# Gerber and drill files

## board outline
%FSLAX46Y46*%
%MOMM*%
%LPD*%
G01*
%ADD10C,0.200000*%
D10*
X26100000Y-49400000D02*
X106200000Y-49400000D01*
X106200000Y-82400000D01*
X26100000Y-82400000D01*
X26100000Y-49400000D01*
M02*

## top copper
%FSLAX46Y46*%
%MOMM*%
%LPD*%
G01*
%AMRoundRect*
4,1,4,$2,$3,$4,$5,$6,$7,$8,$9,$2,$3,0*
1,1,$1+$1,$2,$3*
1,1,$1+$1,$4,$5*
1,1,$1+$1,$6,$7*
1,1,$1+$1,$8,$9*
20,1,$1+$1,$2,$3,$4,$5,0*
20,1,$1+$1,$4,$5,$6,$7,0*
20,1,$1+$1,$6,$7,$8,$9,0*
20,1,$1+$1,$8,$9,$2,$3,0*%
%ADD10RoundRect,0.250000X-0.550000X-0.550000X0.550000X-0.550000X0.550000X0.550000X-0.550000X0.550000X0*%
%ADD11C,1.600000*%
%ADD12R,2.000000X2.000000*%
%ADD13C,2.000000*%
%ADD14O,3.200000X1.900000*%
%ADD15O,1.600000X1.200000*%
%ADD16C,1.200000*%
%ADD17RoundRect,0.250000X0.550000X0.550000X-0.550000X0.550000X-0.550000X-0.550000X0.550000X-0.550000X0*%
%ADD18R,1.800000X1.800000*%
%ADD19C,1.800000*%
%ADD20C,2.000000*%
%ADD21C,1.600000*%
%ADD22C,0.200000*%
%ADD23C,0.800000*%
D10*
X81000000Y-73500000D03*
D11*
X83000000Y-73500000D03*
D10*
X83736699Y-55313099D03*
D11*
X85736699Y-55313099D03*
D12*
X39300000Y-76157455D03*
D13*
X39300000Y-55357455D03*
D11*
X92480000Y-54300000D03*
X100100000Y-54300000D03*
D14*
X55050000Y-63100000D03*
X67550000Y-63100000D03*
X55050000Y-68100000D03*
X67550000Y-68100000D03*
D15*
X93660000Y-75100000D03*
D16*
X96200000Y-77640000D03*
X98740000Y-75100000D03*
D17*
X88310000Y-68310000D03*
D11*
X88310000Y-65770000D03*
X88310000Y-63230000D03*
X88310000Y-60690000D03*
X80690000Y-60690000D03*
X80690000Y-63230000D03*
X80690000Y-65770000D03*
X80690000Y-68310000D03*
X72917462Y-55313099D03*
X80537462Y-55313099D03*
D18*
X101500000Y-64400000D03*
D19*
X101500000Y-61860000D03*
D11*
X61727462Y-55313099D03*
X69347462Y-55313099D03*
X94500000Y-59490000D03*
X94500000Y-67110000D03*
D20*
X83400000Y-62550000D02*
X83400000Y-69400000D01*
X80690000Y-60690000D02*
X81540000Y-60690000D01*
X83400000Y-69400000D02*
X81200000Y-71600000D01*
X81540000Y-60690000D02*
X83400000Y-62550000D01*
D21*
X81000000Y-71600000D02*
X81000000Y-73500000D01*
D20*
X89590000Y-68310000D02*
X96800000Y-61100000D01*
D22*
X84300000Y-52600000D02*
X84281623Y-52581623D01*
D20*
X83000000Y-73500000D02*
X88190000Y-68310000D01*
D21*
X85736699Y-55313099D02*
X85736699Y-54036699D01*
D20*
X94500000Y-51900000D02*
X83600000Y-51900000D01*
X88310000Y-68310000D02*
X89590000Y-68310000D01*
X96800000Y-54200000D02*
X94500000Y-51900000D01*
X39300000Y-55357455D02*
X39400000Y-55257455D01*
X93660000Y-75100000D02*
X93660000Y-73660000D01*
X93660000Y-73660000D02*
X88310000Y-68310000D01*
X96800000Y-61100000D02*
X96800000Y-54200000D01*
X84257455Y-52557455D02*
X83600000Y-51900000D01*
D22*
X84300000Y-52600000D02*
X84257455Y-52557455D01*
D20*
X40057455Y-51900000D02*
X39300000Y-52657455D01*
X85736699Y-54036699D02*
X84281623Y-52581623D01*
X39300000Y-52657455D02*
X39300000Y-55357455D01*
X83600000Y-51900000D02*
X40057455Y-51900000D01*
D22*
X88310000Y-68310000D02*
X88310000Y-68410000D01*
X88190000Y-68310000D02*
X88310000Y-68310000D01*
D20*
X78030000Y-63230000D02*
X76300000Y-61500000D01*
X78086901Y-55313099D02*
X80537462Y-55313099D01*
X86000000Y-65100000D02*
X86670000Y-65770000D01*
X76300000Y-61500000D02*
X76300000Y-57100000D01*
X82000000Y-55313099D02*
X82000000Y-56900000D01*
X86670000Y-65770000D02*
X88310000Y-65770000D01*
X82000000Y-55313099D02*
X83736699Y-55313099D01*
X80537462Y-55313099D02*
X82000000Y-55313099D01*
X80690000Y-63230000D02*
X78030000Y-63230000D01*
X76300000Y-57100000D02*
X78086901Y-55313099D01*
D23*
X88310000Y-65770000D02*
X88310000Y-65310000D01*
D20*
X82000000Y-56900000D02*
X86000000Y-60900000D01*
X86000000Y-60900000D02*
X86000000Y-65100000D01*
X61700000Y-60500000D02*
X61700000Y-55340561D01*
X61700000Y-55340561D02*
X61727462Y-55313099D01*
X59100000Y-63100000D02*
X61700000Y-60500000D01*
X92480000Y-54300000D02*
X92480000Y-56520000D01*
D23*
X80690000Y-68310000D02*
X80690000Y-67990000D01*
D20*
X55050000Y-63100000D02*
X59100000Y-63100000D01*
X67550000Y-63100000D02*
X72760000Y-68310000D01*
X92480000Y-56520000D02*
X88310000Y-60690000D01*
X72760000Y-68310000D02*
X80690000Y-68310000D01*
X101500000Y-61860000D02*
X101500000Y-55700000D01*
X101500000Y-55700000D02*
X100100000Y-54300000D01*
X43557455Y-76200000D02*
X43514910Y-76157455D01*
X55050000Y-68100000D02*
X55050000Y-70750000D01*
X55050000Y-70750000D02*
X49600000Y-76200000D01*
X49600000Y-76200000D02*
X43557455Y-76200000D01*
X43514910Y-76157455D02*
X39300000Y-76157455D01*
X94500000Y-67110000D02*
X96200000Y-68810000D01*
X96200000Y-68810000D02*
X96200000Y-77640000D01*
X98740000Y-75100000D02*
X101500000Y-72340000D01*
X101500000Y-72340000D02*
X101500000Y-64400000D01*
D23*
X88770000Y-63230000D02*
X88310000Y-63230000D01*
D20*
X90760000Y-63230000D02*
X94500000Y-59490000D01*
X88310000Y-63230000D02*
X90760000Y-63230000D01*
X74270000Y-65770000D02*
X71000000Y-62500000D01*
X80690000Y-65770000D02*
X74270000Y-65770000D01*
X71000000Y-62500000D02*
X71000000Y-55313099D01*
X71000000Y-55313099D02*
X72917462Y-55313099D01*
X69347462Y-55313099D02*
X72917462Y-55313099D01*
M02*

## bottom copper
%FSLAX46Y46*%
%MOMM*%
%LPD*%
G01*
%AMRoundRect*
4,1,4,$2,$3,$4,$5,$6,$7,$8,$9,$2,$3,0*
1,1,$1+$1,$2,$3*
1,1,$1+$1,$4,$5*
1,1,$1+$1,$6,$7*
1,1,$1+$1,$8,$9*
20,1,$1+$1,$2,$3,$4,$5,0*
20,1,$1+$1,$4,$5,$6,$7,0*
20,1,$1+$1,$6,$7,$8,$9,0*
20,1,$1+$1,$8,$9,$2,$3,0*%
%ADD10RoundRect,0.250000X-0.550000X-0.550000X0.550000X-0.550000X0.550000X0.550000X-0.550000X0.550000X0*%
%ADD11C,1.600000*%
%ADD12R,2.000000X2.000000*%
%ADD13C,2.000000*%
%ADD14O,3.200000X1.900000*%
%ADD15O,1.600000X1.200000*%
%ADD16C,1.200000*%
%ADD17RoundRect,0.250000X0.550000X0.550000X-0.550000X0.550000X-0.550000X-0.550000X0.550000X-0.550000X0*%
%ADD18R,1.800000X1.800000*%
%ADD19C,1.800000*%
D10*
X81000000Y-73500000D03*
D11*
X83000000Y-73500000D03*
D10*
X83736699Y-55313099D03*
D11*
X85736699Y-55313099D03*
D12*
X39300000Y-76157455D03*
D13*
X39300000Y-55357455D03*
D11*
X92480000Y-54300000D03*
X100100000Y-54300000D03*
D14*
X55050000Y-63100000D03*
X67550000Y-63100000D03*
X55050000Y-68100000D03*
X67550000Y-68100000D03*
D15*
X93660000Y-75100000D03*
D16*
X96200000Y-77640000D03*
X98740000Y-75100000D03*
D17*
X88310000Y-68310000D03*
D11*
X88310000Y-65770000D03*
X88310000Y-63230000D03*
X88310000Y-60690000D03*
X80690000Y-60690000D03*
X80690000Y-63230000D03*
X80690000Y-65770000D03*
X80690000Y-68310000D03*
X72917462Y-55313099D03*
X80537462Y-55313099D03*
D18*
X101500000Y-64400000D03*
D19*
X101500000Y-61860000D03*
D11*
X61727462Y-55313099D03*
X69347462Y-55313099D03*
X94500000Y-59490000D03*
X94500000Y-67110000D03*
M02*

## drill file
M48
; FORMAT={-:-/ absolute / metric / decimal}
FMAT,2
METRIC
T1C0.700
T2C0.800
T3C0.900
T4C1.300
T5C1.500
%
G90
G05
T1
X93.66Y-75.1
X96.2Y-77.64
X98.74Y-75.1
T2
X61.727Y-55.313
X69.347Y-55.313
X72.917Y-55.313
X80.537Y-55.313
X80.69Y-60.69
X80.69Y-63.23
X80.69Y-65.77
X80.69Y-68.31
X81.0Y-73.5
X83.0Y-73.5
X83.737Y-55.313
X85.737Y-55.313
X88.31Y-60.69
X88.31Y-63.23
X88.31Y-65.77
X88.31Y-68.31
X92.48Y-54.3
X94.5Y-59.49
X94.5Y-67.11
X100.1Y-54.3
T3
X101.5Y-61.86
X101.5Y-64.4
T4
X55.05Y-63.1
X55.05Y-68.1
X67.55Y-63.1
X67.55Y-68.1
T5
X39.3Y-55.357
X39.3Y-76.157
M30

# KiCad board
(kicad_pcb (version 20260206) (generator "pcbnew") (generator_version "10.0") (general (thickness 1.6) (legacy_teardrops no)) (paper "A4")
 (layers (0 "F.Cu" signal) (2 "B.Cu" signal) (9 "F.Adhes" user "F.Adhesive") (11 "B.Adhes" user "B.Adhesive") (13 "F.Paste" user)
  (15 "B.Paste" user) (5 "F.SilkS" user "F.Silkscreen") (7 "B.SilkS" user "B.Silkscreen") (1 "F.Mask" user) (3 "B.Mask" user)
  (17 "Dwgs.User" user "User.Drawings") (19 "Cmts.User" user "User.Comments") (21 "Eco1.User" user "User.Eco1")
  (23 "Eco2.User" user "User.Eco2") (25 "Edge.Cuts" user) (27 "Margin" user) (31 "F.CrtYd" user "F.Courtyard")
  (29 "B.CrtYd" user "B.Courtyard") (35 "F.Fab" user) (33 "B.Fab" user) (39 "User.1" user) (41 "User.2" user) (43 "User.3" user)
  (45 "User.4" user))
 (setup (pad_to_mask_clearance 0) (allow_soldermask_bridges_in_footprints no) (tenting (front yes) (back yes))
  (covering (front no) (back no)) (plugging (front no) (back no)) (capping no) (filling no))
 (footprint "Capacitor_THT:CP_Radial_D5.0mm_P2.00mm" (layer "F.Cu") (at 81 73.5)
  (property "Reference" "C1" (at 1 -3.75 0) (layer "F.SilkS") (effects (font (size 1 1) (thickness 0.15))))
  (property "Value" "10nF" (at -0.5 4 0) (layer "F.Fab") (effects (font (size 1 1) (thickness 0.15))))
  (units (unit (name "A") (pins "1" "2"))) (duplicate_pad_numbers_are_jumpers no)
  (pad "1" thru_hole roundrect (at 0 0) (size 1.6 1.6) (drill 0.8) (layers "*.Cu" "*.Mask") (remove_unused_layers no)
   (roundrect_rratio 0.15625) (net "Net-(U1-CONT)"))
  (pad "2" thru_hole circle (at 2 0) (size 1.6 1.6) (drill 0.8) (layers "*.Cu" "*.Mask") (remove_unused_layers no) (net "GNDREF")))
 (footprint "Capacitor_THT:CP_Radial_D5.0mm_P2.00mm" (layer "F.Cu") (at 83.736699 55.313099)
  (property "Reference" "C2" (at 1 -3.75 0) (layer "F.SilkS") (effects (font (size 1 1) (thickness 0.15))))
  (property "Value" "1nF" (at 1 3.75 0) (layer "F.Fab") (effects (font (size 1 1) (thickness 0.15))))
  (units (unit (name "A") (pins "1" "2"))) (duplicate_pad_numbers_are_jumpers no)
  (pad "1" thru_hole roundrect (at 0 0) (size 1.6 1.6) (drill 0.8) (layers "*.Cu" "*.Mask") (remove_unused_layers no)
   (roundrect_rratio 0.15625) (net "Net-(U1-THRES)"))
  (pad "2" thru_hole circle (at 2 0) (size 1.6 1.6) (drill 0.8) (layers "*.Cu" "*.Mask") (remove_unused_layers no) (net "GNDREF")))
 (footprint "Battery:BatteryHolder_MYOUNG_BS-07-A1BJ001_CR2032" (layer "F.Cu") (at 39.3 76.157455 90)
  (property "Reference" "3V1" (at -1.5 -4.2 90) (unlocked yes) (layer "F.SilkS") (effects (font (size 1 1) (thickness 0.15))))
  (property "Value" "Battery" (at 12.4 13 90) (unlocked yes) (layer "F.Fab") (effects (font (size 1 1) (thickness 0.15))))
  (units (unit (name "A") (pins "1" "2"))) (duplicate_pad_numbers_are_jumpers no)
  (pad "1" thru_hole rect (at 0 0 270) (size 2 2) (drill 1.5) (layers "*.Cu" "*.Mask") (remove_unused_layers no) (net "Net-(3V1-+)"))
  (pad "2" thru_hole circle (at 20.8 0 270) (size 2 2) (drill 1.5) (layers "*.Cu" "*.Mask") (remove_unused_layers no) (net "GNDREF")))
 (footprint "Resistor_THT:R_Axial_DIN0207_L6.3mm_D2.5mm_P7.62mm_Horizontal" (layer "F.Cu") (at 92.48 54.3)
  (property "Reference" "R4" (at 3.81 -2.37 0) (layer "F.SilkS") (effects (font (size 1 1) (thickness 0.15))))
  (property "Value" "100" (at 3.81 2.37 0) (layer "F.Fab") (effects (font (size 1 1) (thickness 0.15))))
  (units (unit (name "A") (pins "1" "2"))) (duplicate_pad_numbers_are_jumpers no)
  (pad "1" thru_hole circle (at 0 0) (size 1.6 1.6) (drill 0.8) (layers "*.Cu" "*.Mask") (remove_unused_layers no) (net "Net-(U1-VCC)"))
  (pad "2" thru_hole circle (at 7.62 0) (size 1.6 1.6) (drill 0.8) (layers "*.Cu" "*.Mask") (remove_unused_layers no) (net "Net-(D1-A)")))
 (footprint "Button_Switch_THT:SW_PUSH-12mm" (layer "F.Cu") (at 55.05 63.1)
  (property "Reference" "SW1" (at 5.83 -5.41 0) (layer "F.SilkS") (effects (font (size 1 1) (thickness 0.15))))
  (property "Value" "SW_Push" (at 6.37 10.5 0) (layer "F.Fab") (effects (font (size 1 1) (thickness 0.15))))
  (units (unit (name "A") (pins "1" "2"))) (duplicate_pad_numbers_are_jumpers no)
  (pad "1" thru_hole oval (at 0 0) (size 3.2 1.9) (drill 1.3) (layers "*.Cu" "*.Mask") (remove_unused_layers no) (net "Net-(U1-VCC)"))
  (pad "1" thru_hole oval (at 12.5 0) (size 3.2 1.9) (drill 1.3) (layers "*.Cu" "*.Mask") (remove_unused_layers no) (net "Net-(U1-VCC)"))
  (pad "2" thru_hole oval (at 0 5) (size 3.2 1.9) (drill 1.3) (layers "*.Cu" "*.Mask") (remove_unused_layers no) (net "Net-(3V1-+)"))
  (pad "2" thru_hole oval (at 12.5 5) (size 3.2 1.9) (drill 1.3) (layers "*.Cu" "*.Mask") (remove_unused_layers no) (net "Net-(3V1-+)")))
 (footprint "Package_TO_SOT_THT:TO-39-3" (layer "F.Cu") (at 93.66 75.1)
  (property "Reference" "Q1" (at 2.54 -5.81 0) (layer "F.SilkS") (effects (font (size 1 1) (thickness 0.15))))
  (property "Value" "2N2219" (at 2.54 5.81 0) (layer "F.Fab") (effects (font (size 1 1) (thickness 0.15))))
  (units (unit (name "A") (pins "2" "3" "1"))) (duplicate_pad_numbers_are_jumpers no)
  (pad "1" thru_hole oval (at 0 0) (size 1.6 1.2) (drill 0.7) (layers "*.Cu" "*.Mask") (remove_unused_layers no) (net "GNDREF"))
  (pad "2" thru_hole circle (at 2.54 2.54) (size 1.2 1.2) (drill 0.7) (layers "*.Cu" "*.Mask") (remove_unused_layers no) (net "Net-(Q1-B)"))
  (pad "3" thru_hole circle (at 5.08 0) (size 1.2 1.2) (drill 0.7) (layers "*.Cu" "*.Mask") (remove_unused_layers no) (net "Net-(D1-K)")))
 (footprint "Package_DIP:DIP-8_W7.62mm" (layer "F.Cu") (at 88.31 68.31 180)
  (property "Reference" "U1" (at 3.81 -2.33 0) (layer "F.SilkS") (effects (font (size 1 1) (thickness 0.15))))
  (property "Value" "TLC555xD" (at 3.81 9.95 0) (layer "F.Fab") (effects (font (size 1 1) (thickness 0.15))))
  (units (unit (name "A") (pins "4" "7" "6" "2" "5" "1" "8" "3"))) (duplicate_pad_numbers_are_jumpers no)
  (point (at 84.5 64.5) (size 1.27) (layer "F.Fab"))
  (pad "1" thru_hole roundrect (at 0 0 180) (size 1.6 1.6) (drill 0.8) (layers "*.Cu" "*.Mask") (remove_unused_layers no)
   (roundrect_rratio 0.15625) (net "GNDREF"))
  (pad "2" thru_hole circle (at 0 2.54 180) (size 1.6 1.6) (drill 0.8) (layers "*.Cu" "*.Mask") (remove_unused_layers no)
   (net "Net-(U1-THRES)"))
  (pad "3" thru_hole circle (at 0 5.08 180) (size 1.6 1.6) (drill 0.8) (layers "*.Cu" "*.Mask") (remove_unused_layers no)
   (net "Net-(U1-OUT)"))
  (pad "4" thru_hole circle (at 0 7.62 180) (size 1.6 1.6) (drill 0.8) (layers "*.Cu" "*.Mask") (remove_unused_layers no)
   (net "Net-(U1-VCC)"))
  (pad "5" thru_hole circle (at 7.62 7.62 180) (size 1.6 1.6) (drill 0.8) (layers "*.Cu" "*.Mask") (remove_unused_layers no)
   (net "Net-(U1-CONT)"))
  (pad "6" thru_hole circle (at 7.62 5.08 180) (size 1.6 1.6) (drill 0.8) (layers "*.Cu" "*.Mask") (remove_unused_layers no)
   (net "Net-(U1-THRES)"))
  (pad "7" thru_hole circle (at 7.62 2.54 180) (size 1.6 1.6) (drill 0.8) (layers "*.Cu" "*.Mask") (remove_unused_layers no)
   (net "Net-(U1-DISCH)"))
  (pad "8" thru_hole circle (at 7.62 0 180) (size 1.6 1.6) (drill 0.8) (layers "*.Cu" "*.Mask") (remove_unused_layers no)
   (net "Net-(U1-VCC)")))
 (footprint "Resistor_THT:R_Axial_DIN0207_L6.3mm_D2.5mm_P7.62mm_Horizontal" (layer "F.Cu") (at 72.917462 55.313099)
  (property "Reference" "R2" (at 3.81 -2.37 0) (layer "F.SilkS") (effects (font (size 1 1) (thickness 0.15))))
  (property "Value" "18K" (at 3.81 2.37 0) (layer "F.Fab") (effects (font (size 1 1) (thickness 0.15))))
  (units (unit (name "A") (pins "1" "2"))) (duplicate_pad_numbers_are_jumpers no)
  (pad "1" thru_hole circle (at 0 0) (size 1.6 1.6) (drill 0.8) (layers "*.Cu" "*.Mask") (remove_unused_layers no) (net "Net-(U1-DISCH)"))
  (pad "2" thru_hole circle (at 7.62 0) (size 1.6 1.6) (drill 0.8) (layers "*.Cu" "*.Mask") (remove_unused_layers no) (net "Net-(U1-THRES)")))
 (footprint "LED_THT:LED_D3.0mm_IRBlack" (layer "F.Cu") (at 101.5 64.4 90)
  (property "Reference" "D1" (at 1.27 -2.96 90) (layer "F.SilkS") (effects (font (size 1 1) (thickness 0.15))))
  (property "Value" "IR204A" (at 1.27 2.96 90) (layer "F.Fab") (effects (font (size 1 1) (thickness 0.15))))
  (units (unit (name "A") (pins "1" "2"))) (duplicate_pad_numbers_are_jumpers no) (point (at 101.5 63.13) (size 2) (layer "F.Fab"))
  (pad "1" thru_hole rect (at 0 0 90) (size 1.8 1.8) (drill 0.9) (layers "*.Cu" "*.Mask") (remove_unused_layers no) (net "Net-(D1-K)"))
  (pad "2" thru_hole circle (at 2.54 0 90) (size 1.8 1.8) (drill 0.9) (layers "*.Cu" "*.Mask") (remove_unused_layers no) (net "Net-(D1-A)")))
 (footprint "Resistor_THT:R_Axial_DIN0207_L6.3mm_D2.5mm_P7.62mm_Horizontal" (layer "F.Cu") (at 61.727462 55.313099)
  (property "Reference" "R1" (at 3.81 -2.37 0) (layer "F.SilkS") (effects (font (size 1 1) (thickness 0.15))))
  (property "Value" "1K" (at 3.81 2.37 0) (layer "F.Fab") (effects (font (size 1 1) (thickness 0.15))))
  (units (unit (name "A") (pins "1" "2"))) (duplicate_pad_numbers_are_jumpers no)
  (pad "1" thru_hole circle (at 0 0) (size 1.6 1.6) (drill 0.8) (layers "*.Cu" "*.Mask") (remove_unused_layers no) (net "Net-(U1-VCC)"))
  (pad "2" thru_hole circle (at 7.62 0) (size 1.6 1.6) (drill 0.8) (layers "*.Cu" "*.Mask") (remove_unused_layers no) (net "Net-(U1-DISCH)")))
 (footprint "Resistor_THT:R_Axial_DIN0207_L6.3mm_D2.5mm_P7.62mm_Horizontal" (layer "F.Cu") (at 94.5 59.49 -90)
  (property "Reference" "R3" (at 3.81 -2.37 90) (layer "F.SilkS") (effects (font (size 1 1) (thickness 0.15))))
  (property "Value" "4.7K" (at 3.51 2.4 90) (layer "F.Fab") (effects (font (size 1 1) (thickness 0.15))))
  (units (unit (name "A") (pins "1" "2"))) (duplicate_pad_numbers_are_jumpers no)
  (pad "1" thru_hole circle (at 0 0 270) (size 1.6 1.6) (drill 0.8) (layers "*.Cu" "*.Mask") (remove_unused_layers no) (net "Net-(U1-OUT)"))
  (pad "2" thru_hole circle (at 7.62 0 270) (size 1.6 1.6) (drill 0.8) (layers "*.Cu" "*.Mask") (remove_unused_layers no) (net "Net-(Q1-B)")))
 (gr_rect (start 26.1 49.4) (end 106.2 82.4) (stroke (width 0.2) (type default)) (fill no) (layer "Edge.Cuts"))
 (segment (start 83.4 62.55) (end 83.4 69.4) (width 2) (layer "F.Cu") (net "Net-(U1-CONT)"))
 (segment (start 80.69 60.69) (end 81.54 60.69) (width 2) (layer "F.Cu") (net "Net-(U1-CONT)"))
 (segment (start 83.4 69.4) (end 81.2 71.6) (width 2) (layer "F.Cu") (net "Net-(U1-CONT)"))
 (segment (start 81.54 60.69) (end 83.4 62.55) (width 2) (layer "F.Cu") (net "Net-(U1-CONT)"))
 (segment (start 81 71.6) (end 81 73.5) (width 1.6) (layer "F.Cu") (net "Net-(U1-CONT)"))
 (segment (start 89.59 68.31) (end 96.8 61.1) (width 2) (layer "F.Cu") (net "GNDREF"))
 (segment (start 84.3 52.6) (end 84.281623 52.581623) (width 0.2) (layer "F.Cu") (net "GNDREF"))
 (segment (start 83 73.5) (end 88.19 68.31) (width 2) (layer "F.Cu") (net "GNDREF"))
 (segment (start 85.736699 55.313099) (end 85.736699 54.036699) (width 1.6) (layer "F.Cu") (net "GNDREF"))
 (segment (start 94.5 51.9) (end 83.6 51.9) (width 2) (layer "F.Cu") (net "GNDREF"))
 (segment (start 88.31 68.31) (end 89.59 68.31) (width 2) (layer "F.Cu") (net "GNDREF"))
 (segment (start 96.8 54.2) (end 94.5 51.9) (width 2) (layer "F.Cu") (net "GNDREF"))
 (segment (start 39.3 55.357455) (end 39.4 55.257455) (width 2) (layer "F.Cu") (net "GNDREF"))
 (segment (start 93.66 75.1) (end 93.66 73.66) (width 2) (layer "F.Cu") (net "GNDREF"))
 (segment (start 93.66 73.66) (end 88.31 68.31) (width 2) (layer "F.Cu") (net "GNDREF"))
 (segment (start 96.8 61.1) (end 96.8 54.2) (width 2) (layer "F.Cu") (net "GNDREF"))
 (segment (start 84.257455 52.557455) (end 83.6 51.9) (width 2) (layer "F.Cu") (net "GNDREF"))
 (segment (start 84.3 52.6) (end 84.257455 52.557455) (width 0.2) (layer "F.Cu") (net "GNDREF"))
 (segment (start 40.057455 51.9) (end 39.3 52.657455) (width 2) (layer "F.Cu") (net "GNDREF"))
 (segment (start 85.736699 54.036699) (end 84.281623 52.581623) (width 2) (layer "F.Cu") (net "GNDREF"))
 (segment (start 39.3 52.657455) (end 39.3 55.357455) (width 2) (layer "F.Cu") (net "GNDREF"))
 (segment (start 83.6 51.9) (end 40.057455 51.9) (width 2) (layer "F.Cu") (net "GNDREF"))
 (segment (start 88.31 68.31) (end 88.31 68.41) (width 0.2) (layer "F.Cu") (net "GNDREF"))
 (segment (start 88.19 68.31) (end 88.31 68.31) (width 0.2) (layer "F.Cu") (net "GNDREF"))
 (segment (start 78.03 63.23) (end 76.3 61.5) (width 2) (layer "F.Cu") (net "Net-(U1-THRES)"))
 (segment (start 78.086901 55.313099) (end 80.537462 55.313099) (width 2) (layer "F.Cu") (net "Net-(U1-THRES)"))
 (segment (start 86 65.1) (end 86.67 65.77) (width 2) (layer "F.Cu") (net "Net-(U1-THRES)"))
 (segment (start 76.3 61.5) (end 76.3 57.1) (width 2) (layer "F.Cu") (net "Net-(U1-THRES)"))
 (segment (start 82 55.313099) (end 82 56.9) (width 2) (layer "F.Cu") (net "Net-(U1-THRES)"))
 (segment (start 86.67 65.77) (end 88.31 65.77) (width 2) (layer "F.Cu") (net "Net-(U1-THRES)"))
 (segment (start 82 55.313099) (end 83.736699 55.313099) (width 2) (layer "F.Cu") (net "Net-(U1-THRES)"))
 (segment (start 80.537462 55.313099) (end 82 55.313099) (width 2) (layer "F.Cu") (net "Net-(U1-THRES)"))
 (segment (start 80.69 63.23) (end 78.03 63.23) (width 2) (layer "F.Cu") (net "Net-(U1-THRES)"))
 (segment (start 76.3 57.1) (end 78.086901 55.313099) (width 2) (layer "F.Cu") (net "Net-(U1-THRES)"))
 (segment (start 88.31 65.77) (end 88.31 65.31) (width 0.8) (layer "F.Cu") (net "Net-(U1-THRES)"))
 (segment (start 82 56.9) (end 86 60.9) (width 2) (layer "F.Cu") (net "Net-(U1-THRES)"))
 (segment (start 86 60.9) (end 86 65.1) (width 2) (layer "F.Cu") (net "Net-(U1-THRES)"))
 (segment (start 61.7 60.5) (end 61.7 55.340561) (width 2) (layer "F.Cu") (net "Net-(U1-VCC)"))
 (segment (start 61.7 55.340561) (end 61.727462 55.313099) (width 2) (layer "F.Cu") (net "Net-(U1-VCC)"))
 (segment (start 59.1 63.1) (end 61.7 60.5) (width 2) (layer "F.Cu") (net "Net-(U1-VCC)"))
 (segment (start 92.48 54.3) (end 92.48 56.52) (width 2) (layer "F.Cu") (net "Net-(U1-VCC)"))
 (segment (start 80.69 68.31) (end 80.69 67.99) (width 0.8) (layer "F.Cu") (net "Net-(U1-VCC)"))
 (segment (start 55.05 63.1) (end 59.1 63.1) (width 2) (layer "F.Cu") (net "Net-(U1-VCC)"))
 (segment (start 67.55 63.1) (end 72.76 68.31) (width 2) (layer "F.Cu") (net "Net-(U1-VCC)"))
 (segment (start 92.48 56.52) (end 88.31 60.69) (width 2) (layer "F.Cu") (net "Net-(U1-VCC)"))
 (segment (start 72.76 68.31) (end 80.69 68.31) (width 2) (layer "F.Cu") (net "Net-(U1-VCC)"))
 (segment (start 101.5 61.86) (end 101.5 55.7) (width 2) (layer "F.Cu") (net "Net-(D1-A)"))
 (segment (start 101.5 55.7) (end 100.1 54.3) (width 2) (layer "F.Cu") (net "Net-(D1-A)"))
 (segment (start 43.557455 76.2) (end 43.51491 76.157455) (width 2) (layer "F.Cu") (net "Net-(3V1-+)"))
 (segment (start 55.05 68.1) (end 55.05 70.75) (width 2) (layer "F.Cu") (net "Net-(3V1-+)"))
 (segment (start 55.05 70.75) (end 49.6 76.2) (width 2) (layer "F.Cu") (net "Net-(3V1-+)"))
 (segment (start 49.6 76.2) (end 43.557455 76.2) (width 2) (layer "F.Cu") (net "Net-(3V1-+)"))
 (segment (start 43.51491 76.157455) (end 39.3 76.157455) (width 2) (layer "F.Cu") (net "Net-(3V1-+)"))
 (segment (start 94.5 67.11) (end 96.2 68.81) (width 2) (layer "F.Cu") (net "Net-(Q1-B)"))
 (segment (start 96.2 68.81) (end 96.2 77.64) (width 2) (layer "F.Cu") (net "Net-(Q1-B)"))
 (segment (start 98.74 75.1) (end 101.5 72.34) (width 2) (layer "F.Cu") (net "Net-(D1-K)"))
 (segment (start 101.5 72.34) (end 101.5 64.4) (width 2) (layer "F.Cu") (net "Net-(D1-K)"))
 (segment (start 88.77 63.23) (end 88.31 63.23) (width 0.8) (layer "F.Cu") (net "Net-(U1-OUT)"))
 (segment (start 90.76 63.23) (end 94.5 59.49) (width 2) (layer "F.Cu") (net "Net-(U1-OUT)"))
 (segment (start 88.31 63.23) (end 90.76 63.23) (width 2) (layer "F.Cu") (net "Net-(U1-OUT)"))
 (segment (start 74.27 65.77) (end 71 62.5) (width 2) (layer "F.Cu") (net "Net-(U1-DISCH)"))
 (segment (start 80.69 65.77) (end 74.27 65.77) (width 2) (layer "F.Cu") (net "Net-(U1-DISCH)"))
 (segment (start 71 62.5) (end 71 55.313099) (width 2) (layer "F.Cu") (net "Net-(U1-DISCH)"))
 (segment (start 71 55.313099) (end 72.917462 55.313099) (width 2) (layer "F.Cu") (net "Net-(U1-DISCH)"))
 (segment (start 69.347462 55.313099) (end 72.917462 55.313099) (width 2) (layer "F.Cu") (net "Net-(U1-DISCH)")))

